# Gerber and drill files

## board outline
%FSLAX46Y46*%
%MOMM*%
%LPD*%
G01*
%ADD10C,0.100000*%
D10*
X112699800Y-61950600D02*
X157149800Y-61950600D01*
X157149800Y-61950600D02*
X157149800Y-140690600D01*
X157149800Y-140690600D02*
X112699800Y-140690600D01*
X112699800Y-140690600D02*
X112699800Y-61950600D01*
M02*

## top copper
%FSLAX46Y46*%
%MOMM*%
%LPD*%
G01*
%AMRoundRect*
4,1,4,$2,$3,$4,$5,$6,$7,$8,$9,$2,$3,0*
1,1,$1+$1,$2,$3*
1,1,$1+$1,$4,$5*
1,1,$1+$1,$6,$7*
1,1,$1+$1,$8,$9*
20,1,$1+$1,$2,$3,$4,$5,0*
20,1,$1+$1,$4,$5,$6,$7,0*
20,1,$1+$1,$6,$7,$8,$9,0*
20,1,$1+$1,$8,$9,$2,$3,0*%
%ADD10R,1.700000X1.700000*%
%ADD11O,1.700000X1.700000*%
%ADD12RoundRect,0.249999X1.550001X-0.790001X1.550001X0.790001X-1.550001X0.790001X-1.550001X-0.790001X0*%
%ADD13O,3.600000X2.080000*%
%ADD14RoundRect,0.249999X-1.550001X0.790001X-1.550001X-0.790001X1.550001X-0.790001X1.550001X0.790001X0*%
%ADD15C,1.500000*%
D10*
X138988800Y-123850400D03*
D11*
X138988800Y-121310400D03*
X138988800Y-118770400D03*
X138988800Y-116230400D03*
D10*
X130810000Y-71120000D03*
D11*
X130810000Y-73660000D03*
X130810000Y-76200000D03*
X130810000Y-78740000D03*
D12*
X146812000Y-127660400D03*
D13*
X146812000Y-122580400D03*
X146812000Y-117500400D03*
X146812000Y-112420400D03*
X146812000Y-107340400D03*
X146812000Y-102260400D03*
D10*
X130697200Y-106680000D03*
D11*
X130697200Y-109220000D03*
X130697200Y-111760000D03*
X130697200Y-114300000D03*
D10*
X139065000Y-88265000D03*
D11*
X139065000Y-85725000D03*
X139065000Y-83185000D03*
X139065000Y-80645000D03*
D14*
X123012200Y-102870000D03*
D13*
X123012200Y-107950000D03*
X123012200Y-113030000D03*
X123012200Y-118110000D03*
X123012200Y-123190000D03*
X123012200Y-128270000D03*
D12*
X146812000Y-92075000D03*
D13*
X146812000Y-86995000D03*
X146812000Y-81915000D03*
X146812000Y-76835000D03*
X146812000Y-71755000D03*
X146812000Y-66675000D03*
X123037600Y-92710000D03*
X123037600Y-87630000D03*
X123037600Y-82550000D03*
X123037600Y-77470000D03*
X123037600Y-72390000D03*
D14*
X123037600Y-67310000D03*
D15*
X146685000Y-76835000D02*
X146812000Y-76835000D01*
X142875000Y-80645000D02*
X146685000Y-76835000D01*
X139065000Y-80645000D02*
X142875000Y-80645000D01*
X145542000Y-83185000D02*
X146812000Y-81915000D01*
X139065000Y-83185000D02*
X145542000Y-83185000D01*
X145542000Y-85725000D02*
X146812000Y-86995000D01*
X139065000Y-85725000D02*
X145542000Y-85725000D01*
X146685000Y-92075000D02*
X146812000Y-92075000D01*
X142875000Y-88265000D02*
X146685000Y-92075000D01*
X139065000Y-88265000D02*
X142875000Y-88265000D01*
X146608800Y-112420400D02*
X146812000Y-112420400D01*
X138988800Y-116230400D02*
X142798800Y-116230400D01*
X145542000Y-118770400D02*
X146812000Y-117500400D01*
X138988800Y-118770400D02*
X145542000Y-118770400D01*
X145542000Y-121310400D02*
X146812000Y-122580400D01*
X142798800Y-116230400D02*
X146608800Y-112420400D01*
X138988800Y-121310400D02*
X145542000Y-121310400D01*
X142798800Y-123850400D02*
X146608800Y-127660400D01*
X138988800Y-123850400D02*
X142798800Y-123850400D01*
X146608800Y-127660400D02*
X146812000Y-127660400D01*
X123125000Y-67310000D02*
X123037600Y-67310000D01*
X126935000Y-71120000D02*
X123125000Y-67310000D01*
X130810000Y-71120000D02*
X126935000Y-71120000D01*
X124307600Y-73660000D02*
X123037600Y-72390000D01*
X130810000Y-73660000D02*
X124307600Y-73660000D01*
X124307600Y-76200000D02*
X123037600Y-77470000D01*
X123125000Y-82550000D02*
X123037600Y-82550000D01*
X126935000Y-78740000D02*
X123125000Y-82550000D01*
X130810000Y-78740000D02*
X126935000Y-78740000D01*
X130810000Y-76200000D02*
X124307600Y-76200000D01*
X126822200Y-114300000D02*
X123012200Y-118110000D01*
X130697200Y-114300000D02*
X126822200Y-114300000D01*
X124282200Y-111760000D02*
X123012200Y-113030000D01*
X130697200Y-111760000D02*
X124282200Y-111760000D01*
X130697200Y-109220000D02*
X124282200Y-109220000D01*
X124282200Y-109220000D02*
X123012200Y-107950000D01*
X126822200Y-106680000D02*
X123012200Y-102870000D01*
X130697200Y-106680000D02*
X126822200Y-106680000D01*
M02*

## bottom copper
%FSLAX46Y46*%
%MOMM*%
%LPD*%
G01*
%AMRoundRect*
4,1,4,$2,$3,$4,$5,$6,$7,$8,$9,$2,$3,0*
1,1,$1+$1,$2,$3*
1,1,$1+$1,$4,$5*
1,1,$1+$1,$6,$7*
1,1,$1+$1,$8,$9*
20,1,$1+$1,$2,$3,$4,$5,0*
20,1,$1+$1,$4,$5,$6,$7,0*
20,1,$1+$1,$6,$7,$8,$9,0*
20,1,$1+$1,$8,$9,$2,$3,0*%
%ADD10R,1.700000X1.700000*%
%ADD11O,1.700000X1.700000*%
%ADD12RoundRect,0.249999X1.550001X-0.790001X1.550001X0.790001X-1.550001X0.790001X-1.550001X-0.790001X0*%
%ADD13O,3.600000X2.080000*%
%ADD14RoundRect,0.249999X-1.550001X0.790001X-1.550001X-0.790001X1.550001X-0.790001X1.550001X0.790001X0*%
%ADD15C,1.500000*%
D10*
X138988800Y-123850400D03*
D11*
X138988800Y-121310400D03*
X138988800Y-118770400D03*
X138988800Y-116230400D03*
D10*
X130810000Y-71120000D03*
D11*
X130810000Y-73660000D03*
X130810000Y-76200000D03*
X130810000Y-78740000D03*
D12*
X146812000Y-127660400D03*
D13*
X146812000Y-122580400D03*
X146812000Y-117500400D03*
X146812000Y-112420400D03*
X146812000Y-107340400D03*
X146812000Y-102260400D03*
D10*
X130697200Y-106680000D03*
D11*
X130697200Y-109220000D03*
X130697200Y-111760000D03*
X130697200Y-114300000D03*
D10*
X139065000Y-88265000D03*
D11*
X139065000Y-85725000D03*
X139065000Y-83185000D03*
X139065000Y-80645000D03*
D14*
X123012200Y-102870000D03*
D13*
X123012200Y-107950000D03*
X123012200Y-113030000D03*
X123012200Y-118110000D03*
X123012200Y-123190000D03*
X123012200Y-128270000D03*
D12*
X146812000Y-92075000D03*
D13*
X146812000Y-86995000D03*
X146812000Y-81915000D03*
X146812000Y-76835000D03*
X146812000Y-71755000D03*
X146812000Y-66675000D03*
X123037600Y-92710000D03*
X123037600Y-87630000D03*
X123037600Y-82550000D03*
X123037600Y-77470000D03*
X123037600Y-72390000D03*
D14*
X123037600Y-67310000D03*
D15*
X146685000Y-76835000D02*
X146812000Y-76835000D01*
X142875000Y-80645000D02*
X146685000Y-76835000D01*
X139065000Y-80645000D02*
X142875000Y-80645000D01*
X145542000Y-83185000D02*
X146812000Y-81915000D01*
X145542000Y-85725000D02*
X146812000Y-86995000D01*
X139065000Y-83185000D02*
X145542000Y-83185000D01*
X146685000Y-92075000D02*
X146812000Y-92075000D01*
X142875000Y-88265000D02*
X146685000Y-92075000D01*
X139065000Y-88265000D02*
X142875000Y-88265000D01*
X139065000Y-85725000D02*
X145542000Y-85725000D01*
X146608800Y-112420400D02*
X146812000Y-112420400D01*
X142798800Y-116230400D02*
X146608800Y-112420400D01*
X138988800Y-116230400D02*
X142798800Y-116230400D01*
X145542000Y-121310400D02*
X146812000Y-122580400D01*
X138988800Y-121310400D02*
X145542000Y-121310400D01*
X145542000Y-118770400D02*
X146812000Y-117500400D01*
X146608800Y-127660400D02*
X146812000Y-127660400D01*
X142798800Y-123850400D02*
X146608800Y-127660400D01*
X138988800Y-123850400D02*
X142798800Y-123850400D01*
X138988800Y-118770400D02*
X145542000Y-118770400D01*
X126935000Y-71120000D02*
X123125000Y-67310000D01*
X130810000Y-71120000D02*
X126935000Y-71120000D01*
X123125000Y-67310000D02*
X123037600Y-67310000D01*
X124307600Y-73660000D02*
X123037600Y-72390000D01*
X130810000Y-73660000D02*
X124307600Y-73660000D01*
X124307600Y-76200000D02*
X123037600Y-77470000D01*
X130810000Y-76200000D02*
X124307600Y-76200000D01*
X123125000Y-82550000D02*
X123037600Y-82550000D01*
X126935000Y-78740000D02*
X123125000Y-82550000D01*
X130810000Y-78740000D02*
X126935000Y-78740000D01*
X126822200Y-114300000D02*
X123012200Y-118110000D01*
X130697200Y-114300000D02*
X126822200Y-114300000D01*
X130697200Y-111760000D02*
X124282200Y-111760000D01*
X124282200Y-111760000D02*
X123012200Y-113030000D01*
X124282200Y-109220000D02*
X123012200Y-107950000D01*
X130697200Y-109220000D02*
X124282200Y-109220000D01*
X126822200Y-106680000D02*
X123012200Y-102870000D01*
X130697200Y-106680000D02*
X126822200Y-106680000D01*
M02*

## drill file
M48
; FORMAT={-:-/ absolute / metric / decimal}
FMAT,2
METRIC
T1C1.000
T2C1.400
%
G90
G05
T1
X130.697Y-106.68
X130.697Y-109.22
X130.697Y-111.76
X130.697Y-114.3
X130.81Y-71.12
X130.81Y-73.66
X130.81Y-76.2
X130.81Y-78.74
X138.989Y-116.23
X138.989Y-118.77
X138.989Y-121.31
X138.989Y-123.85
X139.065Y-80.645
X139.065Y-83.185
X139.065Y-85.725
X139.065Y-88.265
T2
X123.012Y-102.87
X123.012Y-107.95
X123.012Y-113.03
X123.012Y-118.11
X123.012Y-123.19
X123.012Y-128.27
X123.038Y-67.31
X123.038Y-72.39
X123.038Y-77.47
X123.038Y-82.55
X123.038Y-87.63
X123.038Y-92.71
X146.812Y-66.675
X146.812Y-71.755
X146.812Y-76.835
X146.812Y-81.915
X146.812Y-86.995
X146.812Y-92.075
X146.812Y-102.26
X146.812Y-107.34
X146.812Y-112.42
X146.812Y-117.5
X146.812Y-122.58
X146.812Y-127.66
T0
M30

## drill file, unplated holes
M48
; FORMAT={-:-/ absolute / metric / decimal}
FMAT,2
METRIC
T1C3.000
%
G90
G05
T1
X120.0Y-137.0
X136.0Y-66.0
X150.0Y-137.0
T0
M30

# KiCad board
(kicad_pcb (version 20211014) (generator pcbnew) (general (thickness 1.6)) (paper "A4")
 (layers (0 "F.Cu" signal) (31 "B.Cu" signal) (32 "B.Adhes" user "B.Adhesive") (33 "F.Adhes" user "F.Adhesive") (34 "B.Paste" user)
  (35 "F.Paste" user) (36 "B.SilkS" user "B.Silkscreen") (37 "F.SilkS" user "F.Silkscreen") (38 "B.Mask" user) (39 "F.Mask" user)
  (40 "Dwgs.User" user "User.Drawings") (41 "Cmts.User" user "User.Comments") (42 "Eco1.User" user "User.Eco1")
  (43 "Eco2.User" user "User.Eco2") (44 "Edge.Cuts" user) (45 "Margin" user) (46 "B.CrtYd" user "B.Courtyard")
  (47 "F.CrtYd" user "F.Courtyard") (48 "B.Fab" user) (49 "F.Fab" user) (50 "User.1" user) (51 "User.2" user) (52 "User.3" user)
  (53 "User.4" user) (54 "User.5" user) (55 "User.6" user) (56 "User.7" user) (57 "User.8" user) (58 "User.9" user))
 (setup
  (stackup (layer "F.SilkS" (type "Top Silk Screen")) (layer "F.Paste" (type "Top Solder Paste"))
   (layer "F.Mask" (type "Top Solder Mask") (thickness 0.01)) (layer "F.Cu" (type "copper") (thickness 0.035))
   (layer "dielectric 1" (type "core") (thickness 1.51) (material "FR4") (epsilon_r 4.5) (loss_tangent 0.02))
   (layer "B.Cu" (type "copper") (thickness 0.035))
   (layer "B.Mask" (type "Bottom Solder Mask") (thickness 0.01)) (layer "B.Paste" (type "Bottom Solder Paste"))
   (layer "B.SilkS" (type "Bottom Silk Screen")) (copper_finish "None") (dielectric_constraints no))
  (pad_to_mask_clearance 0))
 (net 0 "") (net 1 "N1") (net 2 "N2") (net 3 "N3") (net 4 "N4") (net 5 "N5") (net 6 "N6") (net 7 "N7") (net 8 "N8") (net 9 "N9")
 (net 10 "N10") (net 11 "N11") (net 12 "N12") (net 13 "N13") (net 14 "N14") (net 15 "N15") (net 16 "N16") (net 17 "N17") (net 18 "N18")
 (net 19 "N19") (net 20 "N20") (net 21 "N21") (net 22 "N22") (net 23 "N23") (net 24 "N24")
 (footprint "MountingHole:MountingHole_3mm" (layer "F.Cu") (at 136 66)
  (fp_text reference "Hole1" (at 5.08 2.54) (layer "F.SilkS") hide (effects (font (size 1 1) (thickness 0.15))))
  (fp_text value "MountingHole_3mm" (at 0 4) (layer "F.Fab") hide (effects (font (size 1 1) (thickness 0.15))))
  (pad "" np_thru_hole circle (at 0 0) (size 3 3) (drill 3) (layers *.Cu *.Mask)))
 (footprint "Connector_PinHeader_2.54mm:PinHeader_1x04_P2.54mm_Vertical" (layer "F.Cu") (at 138.9888 123.8504 180)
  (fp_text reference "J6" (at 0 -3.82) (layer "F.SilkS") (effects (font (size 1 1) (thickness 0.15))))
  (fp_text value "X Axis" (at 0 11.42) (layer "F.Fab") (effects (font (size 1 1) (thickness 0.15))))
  (pad "1" thru_hole rect (at 0 0 180) (size 1.7 1.7) (drill 1) (layers *.Cu *.Mask) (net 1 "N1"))
  (pad "2" thru_hole oval (at 0 2.54 180) (size 1.7 1.7) (drill 1) (layers *.Cu *.Mask) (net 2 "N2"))
  (pad "3" thru_hole oval (at 0 5.08 180) (size 1.7 1.7) (drill 1) (layers *.Cu *.Mask) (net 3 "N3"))
  (pad "4" thru_hole oval (at 0 7.62 180) (size 1.7 1.7) (drill 1) (layers *.Cu *.Mask) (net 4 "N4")))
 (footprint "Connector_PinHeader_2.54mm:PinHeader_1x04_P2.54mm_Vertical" (layer "F.Cu") (at 130.81 71.12)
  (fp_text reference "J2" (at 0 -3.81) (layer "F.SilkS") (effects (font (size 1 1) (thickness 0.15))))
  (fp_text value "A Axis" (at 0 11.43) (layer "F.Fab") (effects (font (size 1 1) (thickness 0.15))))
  (pad "1" thru_hole rect (at 0 0) (size 1.7 1.7) (drill 1) (layers *.Cu *.Mask) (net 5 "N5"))
  (pad "2" thru_hole oval (at 0 2.54) (size 1.7 1.7) (drill 1) (layers *.Cu *.Mask) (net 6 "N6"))
  (pad "3" thru_hole oval (at 0 5.08) (size 1.7 1.7) (drill 1) (layers *.Cu *.Mask) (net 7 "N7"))
  (pad "4" thru_hole oval (at 0 7.62) (size 1.7 1.7) (drill 1) (layers *.Cu *.Mask) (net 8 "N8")))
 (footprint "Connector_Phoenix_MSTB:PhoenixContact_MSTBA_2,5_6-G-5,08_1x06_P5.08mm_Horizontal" (layer "F.Cu") (at 146.812 127.6604 90)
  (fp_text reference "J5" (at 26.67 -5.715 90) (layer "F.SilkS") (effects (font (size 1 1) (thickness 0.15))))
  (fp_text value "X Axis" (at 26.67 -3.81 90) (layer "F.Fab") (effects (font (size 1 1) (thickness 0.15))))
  (pad "1" thru_hole roundrect (at 0 0 90) (size 2.08 3.6) (drill 1.4) (layers *.Cu *.Mask) (roundrect_rratio 0.1201918269) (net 1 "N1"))
  (pad "2" thru_hole oval (at 5.08 0 90) (size 2.08 3.6) (drill 1.4) (layers *.Cu *.Mask) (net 2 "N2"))
  (pad "3" thru_hole oval (at 10.16 0 90) (size 2.08 3.6) (drill 1.4) (layers *.Cu *.Mask) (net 3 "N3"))
  (pad "4" thru_hole oval (at 15.24 0 90) (size 2.08 3.6) (drill 1.4) (layers *.Cu *.Mask) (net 4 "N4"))
  (pad "5" thru_hole oval (at 20.32 0 90) (size 2.08 3.6) (drill 1.4) (layers *.Cu *.Mask) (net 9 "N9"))
  (pad "6" thru_hole oval (at 25.4 0 90) (size 2.08 3.6) (drill 1.4) (layers *.Cu *.Mask) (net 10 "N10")))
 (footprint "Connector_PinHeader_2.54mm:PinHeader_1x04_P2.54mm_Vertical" (layer "F.Cu") (at 130.6972 106.68)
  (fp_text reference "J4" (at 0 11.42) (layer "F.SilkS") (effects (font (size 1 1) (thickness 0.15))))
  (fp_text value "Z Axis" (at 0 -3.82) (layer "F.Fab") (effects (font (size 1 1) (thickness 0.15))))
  (pad "1" thru_hole rect (at 0 0) (size 1.7 1.7) (drill 1) (layers *.Cu *.Mask) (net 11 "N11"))
  (pad "2" thru_hole oval (at 0 2.54) (size 1.7 1.7) (drill 1) (layers *.Cu *.Mask) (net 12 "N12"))
  (pad "3" thru_hole oval (at 0 5.08) (size 1.7 1.7) (drill 1) (layers *.Cu *.Mask) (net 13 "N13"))
  (pad "4" thru_hole oval (at 0 7.62) (size 1.7 1.7) (drill 1) (layers *.Cu *.Mask) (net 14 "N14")))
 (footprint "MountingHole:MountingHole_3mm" (layer "F.Cu") (at 150 137)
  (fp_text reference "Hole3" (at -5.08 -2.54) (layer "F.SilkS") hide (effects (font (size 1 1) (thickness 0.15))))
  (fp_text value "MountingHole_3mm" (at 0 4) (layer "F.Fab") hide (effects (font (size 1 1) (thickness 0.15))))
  (pad "" np_thru_hole circle (at 0 0) (size 3 3) (drill 3) (layers *.Cu *.Mask)))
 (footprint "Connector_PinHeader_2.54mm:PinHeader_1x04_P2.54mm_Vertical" (layer "F.Cu") (at 139.065 88.265 180)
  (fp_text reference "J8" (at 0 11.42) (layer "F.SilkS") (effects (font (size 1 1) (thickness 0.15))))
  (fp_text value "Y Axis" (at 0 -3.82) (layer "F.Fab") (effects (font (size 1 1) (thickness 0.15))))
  (pad "1" thru_hole rect (at 0 0 180) (size 1.7 1.7) (drill 1) (layers *.Cu *.Mask) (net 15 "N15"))
  (pad "2" thru_hole oval (at 0 2.54 180) (size 1.7 1.7) (drill 1) (layers *.Cu *.Mask) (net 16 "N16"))
  (pad "3" thru_hole oval (at 0 5.08 180) (size 1.7 1.7) (drill 1) (layers *.Cu *.Mask) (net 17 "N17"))
  (pad "4" thru_hole oval (at 0 7.62 180) (size 1.7 1.7) (drill 1) (layers *.Cu *.Mask) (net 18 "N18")))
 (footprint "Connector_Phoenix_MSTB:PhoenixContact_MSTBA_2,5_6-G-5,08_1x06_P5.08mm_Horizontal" (layer "F.Cu") (at 123.0122 102.87 -90)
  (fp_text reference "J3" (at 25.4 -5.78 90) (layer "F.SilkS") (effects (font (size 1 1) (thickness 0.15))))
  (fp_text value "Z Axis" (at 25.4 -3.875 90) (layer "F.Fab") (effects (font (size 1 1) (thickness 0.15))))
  (pad "1" thru_hole roundrect (at 0 0 270) (size 2.08 3.6) (drill 1.4) (layers *.Cu *.Mask) (roundrect_rratio 0.1201918269) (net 11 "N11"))
  (pad "2" thru_hole oval (at 5.08 0 270) (size 2.08 3.6) (drill 1.4) (layers *.Cu *.Mask) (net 12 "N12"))
  (pad "3" thru_hole oval (at 10.16 0 270) (size 2.08 3.6) (drill 1.4) (layers *.Cu *.Mask) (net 13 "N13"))
  (pad "4" thru_hole oval (at 15.24 0 270) (size 2.08 3.6) (drill 1.4) (layers *.Cu *.Mask) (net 14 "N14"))
  (pad "5" thru_hole oval (at 20.32 0 270) (size 2.08 3.6) (drill 1.4) (layers *.Cu *.Mask) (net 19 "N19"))
  (pad "6" thru_hole oval (at 25.4 0 270) (size 2.08 3.6) (drill 1.4) (layers *.Cu *.Mask) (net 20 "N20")))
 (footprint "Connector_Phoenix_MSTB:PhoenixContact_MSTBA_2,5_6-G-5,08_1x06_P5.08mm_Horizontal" (layer "F.Cu") (at 146.812 92.075 90)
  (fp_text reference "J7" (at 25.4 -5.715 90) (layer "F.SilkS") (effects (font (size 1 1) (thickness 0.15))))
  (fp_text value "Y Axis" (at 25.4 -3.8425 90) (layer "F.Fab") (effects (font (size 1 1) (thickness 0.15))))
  (pad "1" thru_hole roundrect (at 0 0 90) (size 2.08 3.6) (drill 1.4) (layers *.Cu *.Mask) (roundrect_rratio 0.1201918269) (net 15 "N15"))
  (pad "2" thru_hole oval (at 5.08 0 90) (size 2.08 3.6) (drill 1.4) (layers *.Cu *.Mask) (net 16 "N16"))
  (pad "3" thru_hole oval (at 10.16 0 90) (size 2.08 3.6) (drill 1.4) (layers *.Cu *.Mask) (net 17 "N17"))
  (pad "4" thru_hole oval (at 15.24 0 90) (size 2.08 3.6) (drill 1.4) (layers *.Cu *.Mask) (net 18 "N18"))
  (pad "5" thru_hole oval (at 20.32 0 90) (size 2.08 3.6) (drill 1.4) (layers *.Cu *.Mask) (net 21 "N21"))
  (pad "6" thru_hole oval (at 25.4 0 90) (size 2.08 3.6) (drill 1.4) (layers *.Cu *.Mask) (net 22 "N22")))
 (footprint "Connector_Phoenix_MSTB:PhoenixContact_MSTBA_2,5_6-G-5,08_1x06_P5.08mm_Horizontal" (layer "F.Cu") (at 123.0376 67.31 -90)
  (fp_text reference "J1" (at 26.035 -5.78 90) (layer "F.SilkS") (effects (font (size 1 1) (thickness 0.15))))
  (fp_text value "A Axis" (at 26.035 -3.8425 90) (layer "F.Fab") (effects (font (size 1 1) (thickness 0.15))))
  (pad "1" thru_hole roundrect (at 0 0 270) (size 2.08 3.6) (drill 1.4) (layers *.Cu *.Mask) (roundrect_rratio 0.1201918269) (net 5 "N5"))
  (pad "2" thru_hole oval (at 5.08 0 270) (size 2.08 3.6) (drill 1.4) (layers *.Cu *.Mask) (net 6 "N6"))
  (pad "3" thru_hole oval (at 10.16 0 270) (size 2.08 3.6) (drill 1.4) (layers *.Cu *.Mask) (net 7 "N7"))
  (pad "4" thru_hole oval (at 15.24 0 270) (size 2.08 3.6) (drill 1.4) (layers *.Cu *.Mask) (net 8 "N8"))
  (pad "5" thru_hole oval (at 20.32 0 270) (size 2.08 3.6) (drill 1.4) (layers *.Cu *.Mask) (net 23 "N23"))
  (pad "6" thru_hole oval (at 25.4 0 270) (size 2.08 3.6) (drill 1.4) (layers *.Cu *.Mask) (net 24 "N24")))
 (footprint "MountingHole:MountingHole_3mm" (layer "F.Cu") (at 120 137)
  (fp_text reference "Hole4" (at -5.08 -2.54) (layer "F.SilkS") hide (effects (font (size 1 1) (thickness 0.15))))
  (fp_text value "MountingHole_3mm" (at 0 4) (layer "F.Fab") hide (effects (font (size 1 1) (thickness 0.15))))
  (pad "" np_thru_hole circle (at 0 0) (size 3 3) (drill 3) (layers *.Cu *.Mask)))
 (gr_rect (start 112.6998 61.9506) (end 157.1498 140.6906) (layer "Edge.Cuts") (width 0.1) (fill none))
 (segment (start 126.935 71.12) (end 123.125 67.31) (width 1.5) (layer "F.Cu") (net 5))
 (segment (start 130.81 71.12) (end 126.935 71.12) (width 1.5) (layer "F.Cu") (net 5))
 (segment (start 123.125 67.31) (end 123.0376 67.31) (width 1.5) (layer "F.Cu") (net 5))
 (segment (start 123.125 67.31) (end 123.0376 67.31) (width 1.5) (layer "B.Cu") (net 5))
 (segment (start 130.81 71.12) (end 126.935 71.12) (width 1.5) (layer "B.Cu") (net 5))
 (segment (start 126.935 71.12) (end 123.125 67.31) (width 1.5) (layer "B.Cu") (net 5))
 (segment (start 130.81 73.66) (end 124.3076 73.66) (width 1.5) (layer "F.Cu") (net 6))
 (segment (start 124.3076 73.66) (end 123.0376 72.39) (width 1.5) (layer "F.Cu") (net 6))
 (segment (start 130.81 73.66) (end 124.3076 73.66) (width 1.5) (layer "B.Cu") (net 6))
 (segment (start 124.3076 73.66) (end 123.0376 72.39) (width 1.5) (layer "B.Cu") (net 6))
 (segment (start 124.3076 76.2) (end 123.0376 77.47) (width 1.5) (layer "F.Cu") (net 7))
 (segment (start 130.81 76.2) (end 124.3076 76.2) (width 1.5) (layer "F.Cu") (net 7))
 (segment (start 130.81 76.2) (end 124.3076 76.2) (width 1.5) (layer "B.Cu") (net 7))
 (segment (start 124.3076 76.2) (end 123.0376 77.47) (width 1.5) (layer "B.Cu") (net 7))
 (segment (start 130.81 78.74) (end 126.935 78.74) (width 1.5) (layer "F.Cu") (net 8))
 (segment (start 123.125 82.55) (end 123.0376 82.55) (width 1.5) (layer "F.Cu") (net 8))
 (segment (start 126.935 78.74) (end 123.125 82.55) (width 1.5) (layer "F.Cu") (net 8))
 (segment (start 123.125 82.55) (end 123.0376 82.55) (width 1.5) (layer "B.Cu") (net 8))
 (segment (start 126.935 78.74) (end 123.125 82.55) (width 1.5) (layer "B.Cu") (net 8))
 (segment (start 130.81 78.74) (end 126.935 78.74) (width 1.5) (layer "B.Cu") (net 8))
 (segment (start 126.8222 106.68) (end 123.0122 102.87) (width 1.5) (layer "F.Cu") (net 11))
 (segment (start 130.6972 106.68) (end 126.8222 106.68) (width 1.5) (layer "F.Cu") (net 11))
 (segment (start 126.8222 106.68) (end 123.0122 102.87) (width 1.5) (layer "B.Cu") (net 11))
 (segment (start 130.6972 106.68) (end 126.8222 106.68) (width 1.5) (layer "B.Cu") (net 11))
 (segment (start 124.2822 109.22) (end 123.0122 107.95) (width 1.5) (layer "F.Cu") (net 12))
 (segment (start 130.6972 109.22) (end 124.2822 109.22) (width 1.5) (layer "F.Cu") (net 12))
 (segment (start 130.6972 109.22) (end 124.2822 109.22) (width 1.5) (layer "B.Cu") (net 12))
 (segment (start 124.2822 109.22) (end 123.0122 107.95) (width 1.5) (layer "B.Cu") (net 12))
 (segment (start 130.6972 111.76) (end 124.2822 111.76) (width 1.5) (layer "F.Cu") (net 13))
 (segment (start 124.2822 111.76) (end 123.0122 113.03) (width 1.5) (layer "F.Cu") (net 13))
 (segment (start 130.6972 111.76) (end 124.2822 111.76) (width 1.5) (layer "B.Cu") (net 13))
 (segment (start 124.2822 111.76) (end 123.0122 113.03) (width 1.5) (layer "B.Cu") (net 13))
 (segment (start 126.8222 114.3) (end 123.0122 118.11) (width 1.5) (layer "F.Cu") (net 14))
 (segment (start 130.6972 114.3) (end 126.8222 114.3) (width 1.5) (layer "F.Cu") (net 14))
 (segment (start 130.6972 114.3) (end 126.8222 114.3) (width 1.5) (layer "B.Cu") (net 14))
 (segment (start 126.8222 114.3) (end 123.0122 118.11) (width 1.5) (layer "B.Cu") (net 14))
 (segment (start 142.7988 123.8504) (end 146.6088 127.6604) (width 1.5) (layer "F.Cu") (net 1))
 (segment (start 138.9888 123.8504) (end 142.7988 123.8504) (width 1.5) (layer "F.Cu") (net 1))
 (segment (start 146.6088 127.6604) (end 146.812 127.6604) (width 1.5) (layer "F.Cu") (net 1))
 (segment (start 138.9888 123.8504) (end 142.7988 123.8504) (width 1.5) (layer "B.Cu") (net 1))
 (segment (start 146.6088 127.6604) (end 146.812 127.6604) (width 1.5) (layer "B.Cu") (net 1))
 (segment (start 142.7988 123.8504) (end 146.6088 127.6604) (width 1.5) (layer "B.Cu") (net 1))
 (segment (start 145.542 121.3104) (end 146.812 122.5804) (width 1.5) (layer "F.Cu") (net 2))
 (segment (start 138.9888 121.3104) (end 145.542 121.3104) (width 1.5) (layer "F.Cu") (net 2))
 (segment (start 145.542 121.3104) (end 146.812 122.5804) (width 1.5) (layer "B.Cu") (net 2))
 (segment (start 138.9888 121.3104) (end 145.542 121.3104) (width 1.5) (layer "B.Cu") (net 2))
 (segment (start 145.542 118.7704) (end 146.812 117.5004) (width 1.5) (layer "F.Cu") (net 3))
 (segment (start 138.9888 118.7704) (end 145.542 118.7704) (width 1.5) (layer "F.Cu") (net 3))
 (segment (start 138.9888 118.7704) (end 145.542 118.7704) (width 1.5) (layer "B.Cu") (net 3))
 (segment (start 145.542 118.7704) (end 146.812 117.5004) (width 1.5) (layer "B.Cu") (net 3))
 (segment (start 138.9888 116.2304) (end 142.7988 116.2304) (width 1.5) (layer "F.Cu") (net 4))
 (segment (start 146.6088 112.4204) (end 146.812 112.4204) (width 1.5) (layer "F.Cu") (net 4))
 (segment (start 142.7988 116.2304) (end 146.6088 112.4204) (width 1.5) (layer "F.Cu") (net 4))
 (segment (start 146.6088 112.4204) (end 146.812 112.4204) (width 1.5) (layer "B.Cu") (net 4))
 (segment (start 138.9888 116.2304) (end 142.7988 116.2304) (width 1.5) (layer "B.Cu") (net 4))
 (segment (start 142.7988 116.2304) (end 146.6088 112.4204) (width 1.5) (layer "B.Cu") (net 4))
 (segment (start 146.685 92.075) (end 146.812 92.075) (width 1.5) (layer "F.Cu") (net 15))
 (segment (start 139.065 88.265) (end 142.875 88.265) (width 1.5) (layer "F.Cu") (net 15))
 (segment (start 142.875 88.265) (end 146.685 92.075) (width 1.5) (layer "F.Cu") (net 15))
 (segment (start 146.685 92.075) (end 146.812 92.075) (width 1.5) (layer "B.Cu") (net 15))
 (segment (start 139.065 88.265) (end 142.875 88.265) (width 1.5) (layer "B.Cu") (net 15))
 (segment (start 142.875 88.265) (end 146.685 92.075) (width 1.5) (layer "B.Cu") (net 15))
 (segment (start 139.065 85.725) (end 145.542 85.725) (width 1.5) (layer "F.Cu") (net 16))
 (segment (start 145.542 85.725) (end 146.812 86.995) (width 1.5) (layer "F.Cu") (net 16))
 (segment (start 139.065 85.725) (end 145.542 85.725) (width 1.5) (layer "B.Cu") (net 16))
 (segment (start 145.542 85.725) (end 146.812 86.995) (width 1.5) (layer "B.Cu") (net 16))
 (segment (start 145.542 83.185) (end 146.812 81.915) (width 1.5) (layer "F.Cu") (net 17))
 (segment (start 139.065 83.185) (end 145.542 83.185) (width 1.5) (layer "F.Cu") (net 17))
 (segment (start 139.065 83.185) (end 145.542 83.185) (width 1.5) (layer "B.Cu") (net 17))
 (segment (start 145.542 83.185) (end 146.812 81.915) (width 1.5) (layer "B.Cu") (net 17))
 (segment (start 139.065 80.645) (end 142.875 80.645) (width 1.5) (layer "F.Cu") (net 18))
 (segment (start 146.685 76.835) (end 146.812 76.835) (width 1.5) (layer "F.Cu") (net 18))
 (segment (start 142.875 80.645) (end 146.685 76.835) (width 1.5) (layer "F.Cu") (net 18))
 (segment (start 139.065 80.645) (end 142.875 80.645) (width 1.5) (layer "B.Cu") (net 18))
 (segment (start 142.875 80.645) (end 146.685 76.835) (width 1.5) (layer "B.Cu") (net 18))
 (segment (start 146.685 76.835) (end 146.812 76.835) (width 1.5) (layer "B.Cu") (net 18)))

